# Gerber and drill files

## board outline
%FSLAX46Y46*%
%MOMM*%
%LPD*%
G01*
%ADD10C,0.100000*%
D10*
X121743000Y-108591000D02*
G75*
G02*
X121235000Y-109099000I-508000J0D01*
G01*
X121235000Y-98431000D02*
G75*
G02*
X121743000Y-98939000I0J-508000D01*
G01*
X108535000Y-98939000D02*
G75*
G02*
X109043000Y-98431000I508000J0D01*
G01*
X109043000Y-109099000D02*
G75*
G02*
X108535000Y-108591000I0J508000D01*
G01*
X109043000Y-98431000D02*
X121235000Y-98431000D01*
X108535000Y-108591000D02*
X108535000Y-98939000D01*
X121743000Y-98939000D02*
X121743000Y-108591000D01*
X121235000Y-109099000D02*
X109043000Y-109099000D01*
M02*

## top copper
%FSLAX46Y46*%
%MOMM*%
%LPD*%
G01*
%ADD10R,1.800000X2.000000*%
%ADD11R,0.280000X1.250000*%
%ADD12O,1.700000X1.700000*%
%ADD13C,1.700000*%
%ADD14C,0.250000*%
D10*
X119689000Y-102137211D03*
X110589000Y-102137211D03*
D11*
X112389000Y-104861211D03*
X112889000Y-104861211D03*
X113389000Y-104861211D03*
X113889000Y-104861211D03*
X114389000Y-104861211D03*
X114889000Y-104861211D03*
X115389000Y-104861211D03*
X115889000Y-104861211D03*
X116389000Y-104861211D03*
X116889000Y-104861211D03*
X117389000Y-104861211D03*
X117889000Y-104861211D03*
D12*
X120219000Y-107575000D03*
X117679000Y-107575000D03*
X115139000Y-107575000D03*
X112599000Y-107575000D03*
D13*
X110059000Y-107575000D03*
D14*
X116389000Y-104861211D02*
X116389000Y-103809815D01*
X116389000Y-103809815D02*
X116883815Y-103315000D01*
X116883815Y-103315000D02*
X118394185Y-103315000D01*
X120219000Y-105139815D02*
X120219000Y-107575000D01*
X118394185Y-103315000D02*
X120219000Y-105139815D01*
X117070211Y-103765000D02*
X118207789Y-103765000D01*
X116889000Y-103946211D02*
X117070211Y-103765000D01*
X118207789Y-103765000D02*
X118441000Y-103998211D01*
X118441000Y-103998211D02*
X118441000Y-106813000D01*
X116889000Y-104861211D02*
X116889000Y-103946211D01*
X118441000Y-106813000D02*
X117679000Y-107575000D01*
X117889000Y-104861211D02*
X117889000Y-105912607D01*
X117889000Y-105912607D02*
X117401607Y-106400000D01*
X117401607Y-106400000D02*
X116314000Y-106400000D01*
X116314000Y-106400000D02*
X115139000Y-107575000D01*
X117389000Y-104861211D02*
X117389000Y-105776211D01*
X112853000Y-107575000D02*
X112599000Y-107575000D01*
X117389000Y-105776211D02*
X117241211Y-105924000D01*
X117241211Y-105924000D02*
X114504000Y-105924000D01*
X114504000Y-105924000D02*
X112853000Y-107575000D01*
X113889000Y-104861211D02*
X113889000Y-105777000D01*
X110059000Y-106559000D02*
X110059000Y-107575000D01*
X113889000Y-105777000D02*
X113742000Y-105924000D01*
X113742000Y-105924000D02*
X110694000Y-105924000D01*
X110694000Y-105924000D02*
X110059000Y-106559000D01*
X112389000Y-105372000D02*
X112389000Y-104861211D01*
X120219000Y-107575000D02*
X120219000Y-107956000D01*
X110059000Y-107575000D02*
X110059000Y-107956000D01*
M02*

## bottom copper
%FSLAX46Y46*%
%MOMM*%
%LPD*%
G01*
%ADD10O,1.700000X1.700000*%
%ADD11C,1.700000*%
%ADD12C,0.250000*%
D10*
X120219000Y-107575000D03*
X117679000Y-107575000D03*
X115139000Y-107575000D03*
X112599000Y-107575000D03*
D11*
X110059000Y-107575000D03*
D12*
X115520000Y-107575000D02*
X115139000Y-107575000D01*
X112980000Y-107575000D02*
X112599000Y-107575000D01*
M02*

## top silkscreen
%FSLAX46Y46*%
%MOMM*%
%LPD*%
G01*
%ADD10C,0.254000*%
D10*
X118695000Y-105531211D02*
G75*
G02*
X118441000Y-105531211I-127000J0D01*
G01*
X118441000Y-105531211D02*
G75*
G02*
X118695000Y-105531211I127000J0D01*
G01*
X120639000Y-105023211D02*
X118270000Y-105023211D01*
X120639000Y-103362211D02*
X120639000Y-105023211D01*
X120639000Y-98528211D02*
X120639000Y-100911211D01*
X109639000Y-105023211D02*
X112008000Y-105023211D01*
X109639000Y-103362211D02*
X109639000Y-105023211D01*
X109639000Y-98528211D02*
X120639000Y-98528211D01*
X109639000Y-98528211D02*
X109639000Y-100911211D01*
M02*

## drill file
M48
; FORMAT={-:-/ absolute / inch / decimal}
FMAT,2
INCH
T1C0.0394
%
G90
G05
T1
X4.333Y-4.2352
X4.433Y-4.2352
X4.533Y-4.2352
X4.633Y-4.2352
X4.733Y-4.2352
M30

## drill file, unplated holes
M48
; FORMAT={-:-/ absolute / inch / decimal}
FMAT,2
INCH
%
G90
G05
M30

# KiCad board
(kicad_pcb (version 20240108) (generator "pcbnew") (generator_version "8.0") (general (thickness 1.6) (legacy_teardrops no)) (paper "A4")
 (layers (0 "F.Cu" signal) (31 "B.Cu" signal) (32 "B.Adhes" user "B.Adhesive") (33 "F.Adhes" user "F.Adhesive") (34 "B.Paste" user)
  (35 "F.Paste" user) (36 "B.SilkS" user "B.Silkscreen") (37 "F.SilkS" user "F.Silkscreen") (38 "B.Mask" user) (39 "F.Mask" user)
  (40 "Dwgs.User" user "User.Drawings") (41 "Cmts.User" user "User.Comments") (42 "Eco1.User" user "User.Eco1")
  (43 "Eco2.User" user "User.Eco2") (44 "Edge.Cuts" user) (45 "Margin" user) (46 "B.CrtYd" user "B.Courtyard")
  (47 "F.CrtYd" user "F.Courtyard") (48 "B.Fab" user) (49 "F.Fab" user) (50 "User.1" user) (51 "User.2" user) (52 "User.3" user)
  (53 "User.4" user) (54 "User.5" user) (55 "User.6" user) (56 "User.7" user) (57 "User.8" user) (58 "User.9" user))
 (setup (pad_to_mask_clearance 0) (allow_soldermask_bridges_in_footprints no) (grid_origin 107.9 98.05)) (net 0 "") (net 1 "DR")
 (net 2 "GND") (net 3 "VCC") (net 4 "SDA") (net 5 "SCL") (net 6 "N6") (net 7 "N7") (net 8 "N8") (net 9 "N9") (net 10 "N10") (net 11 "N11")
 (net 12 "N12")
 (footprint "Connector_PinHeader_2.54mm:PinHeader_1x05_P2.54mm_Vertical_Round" (layer "F.Cu") (at 110.059 107.575 90)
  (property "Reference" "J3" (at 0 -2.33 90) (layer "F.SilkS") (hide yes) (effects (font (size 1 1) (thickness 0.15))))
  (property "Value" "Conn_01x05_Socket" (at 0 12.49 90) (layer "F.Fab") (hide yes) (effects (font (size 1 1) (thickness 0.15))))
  (pad "1" thru_hole circle (at 0 0 90) (size 1.7 1.7) (drill 1) (layers "*.Cu" "*.Mask") (remove_unused_layers no) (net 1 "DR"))
  (pad "2" thru_hole oval (at 0 2.54 90) (size 1.7 1.7) (drill 1) (layers "*.Cu" "*.Mask") (remove_unused_layers no) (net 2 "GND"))
  (pad "3" thru_hole oval (at 0 5.08 90) (size 1.7 1.7) (drill 1) (layers "*.Cu" "*.Mask") (remove_unused_layers no) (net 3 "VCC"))
  (pad "4" thru_hole oval (at 0 7.62 90) (size 1.7 1.7) (drill 1) (layers "*.Cu" "*.Mask") (remove_unused_layers no) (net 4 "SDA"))
  (pad "5" thru_hole oval (at 0 10.16 90) (size 1.7 1.7) (drill 1) (layers "*.Cu" "*.Mask") (remove_unused_layers no) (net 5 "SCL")))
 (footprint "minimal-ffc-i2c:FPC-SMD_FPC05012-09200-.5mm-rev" (layer "F.Cu") (at 115.139 103.499211 180)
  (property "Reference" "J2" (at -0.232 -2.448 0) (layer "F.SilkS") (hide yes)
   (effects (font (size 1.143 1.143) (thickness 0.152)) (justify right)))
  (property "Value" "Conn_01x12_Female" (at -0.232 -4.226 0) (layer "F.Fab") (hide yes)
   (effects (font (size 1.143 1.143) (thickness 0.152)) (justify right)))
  (fp_line (start 5.5 4.971) (end 5.5 2.588) (stroke (width 0.254) (type solid)) (layer "F.SilkS"))
  (fp_line (start 5.5 4.971) (end -5.5 4.971) (stroke (width 0.254) (type solid)) (layer "F.SilkS"))
  (fp_line (start 5.5 0.137) (end 5.5 -1.524) (stroke (width 0.254) (type solid)) (layer "F.SilkS"))
  (fp_line (start 5.5 -1.524) (end 3.131 -1.524) (stroke (width 0.254) (type solid)) (layer "F.SilkS"))
  (fp_line (start -5.5 4.971) (end -5.5 2.588) (stroke (width 0.254) (type solid)) (layer "F.SilkS"))
  (fp_line (start -5.5 0.137) (end -5.5 -1.524) (stroke (width 0.254) (type solid)) (layer "F.SilkS"))
  (fp_line (start -5.5 -1.524) (end -3.131 -1.524) (stroke (width 0.254) (type solid)) (layer "F.SilkS"))
  (fp_circle (center -3.429 -2.032) (end -3.302 -2.032) (stroke (width 0.254) (type solid)) (fill none) (layer "F.SilkS"))
  (pad "1" smd rect (at -2.75 -1.362 180) (size 0.28 1.25) (layers "F.Cu" "F.Paste" "F.Mask") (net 3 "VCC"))
  (pad "2" smd rect (at -2.25 -1.362 180) (size 0.28 1.25) (layers "F.Cu" "F.Paste" "F.Mask") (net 2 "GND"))
  (pad "3" smd rect (at -1.75 -1.362 180) (size 0.28 1.25) (layers "F.Cu" "F.Paste" "F.Mask") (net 4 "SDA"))
  (pad "4" smd rect (at -1.25 -1.362 180) (size 0.28 1.25) (layers "F.Cu" "F.Paste" "F.Mask") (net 5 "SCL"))
  (pad "5" smd rect (at -0.75 -1.362 180) (size 0.28 1.25) (layers "F.Cu" "F.Paste" "F.Mask") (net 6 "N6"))
  (pad "6" smd rect (at -0.25 -1.362 180) (size 0.28 1.25) (layers "F.Cu" "F.Paste" "F.Mask") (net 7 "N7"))
  (pad "7" smd rect (at 0.25 -1.362 180) (size 0.28 1.25) (layers "F.Cu" "F.Paste" "F.Mask") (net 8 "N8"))
  (pad "8" smd rect (at 0.75 -1.362 180) (size 0.28 1.25) (layers "F.Cu" "F.Paste" "F.Mask") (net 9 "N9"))
  (pad "9" smd rect (at 1.25 -1.362 180) (size 0.28 1.25) (layers "F.Cu" "F.Paste" "F.Mask") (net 1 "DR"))
  (pad "10" smd rect (at 1.75 -1.362 180) (size 0.28 1.25) (layers "F.Cu" "F.Paste" "F.Mask") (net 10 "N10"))
  (pad "11" smd rect (at 2.25 -1.362 180) (size 0.28 1.25) (layers "F.Cu" "F.Paste" "F.Mask") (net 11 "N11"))
  (pad "12" smd rect (at 2.75 -1.362 180) (size 0.28 1.25) (layers "F.Cu" "F.Paste" "F.Mask") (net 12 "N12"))
  (pad "13" smd rect (at 4.55 1.362 180) (size 1.8 2) (layers "F.Cu" "F.Paste" "F.Mask"))
  (pad "14" smd rect (at -4.55 1.362 180) (size 1.8 2) (layers "F.Cu" "F.Paste" "F.Mask")))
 (gr_arc (start 121.743 108.591) (mid 121.59421 108.95021) (end 121.235 109.099) (stroke (width 0.1) (type default)) (layer "Edge.Cuts"))
 (gr_arc (start 121.235 98.431) (mid 121.59421 98.57979) (end 121.743 98.939) (stroke (width 0.1) (type default)) (layer "Edge.Cuts"))
 (gr_line (start 121.235 109.099) (end 109.043 109.099) (stroke (width 0.1) (type default)) (layer "Edge.Cuts"))
 (gr_arc (start 109.043 109.099) (mid 108.68379 108.95021) (end 108.535 108.591) (stroke (width 0.1) (type default)) (layer "Edge.Cuts"))
 (gr_line (start 109.043 98.431) (end 121.235 98.431) (stroke (width 0.1) (type default)) (layer "Edge.Cuts"))
 (gr_line (start 121.743 98.939) (end 121.743 108.591) (stroke (width 0.1) (type default)) (layer "Edge.Cuts"))
 (gr_line (start 108.535 108.591) (end 108.535 98.939) (stroke (width 0.1) (type default)) (layer "Edge.Cuts"))
 (gr_arc (start 108.535 98.939) (mid 108.68379 98.57979) (end 109.043 98.431) (stroke (width 0.1) (type default)) (layer "Edge.Cuts"))
 (segment (start 116.314 106.4) (end 115.139 107.575) (width 0.25) (layer "F.Cu") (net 3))
 (segment (start 117.401607 106.4) (end 116.314 106.4) (width 0.25) (layer "F.Cu") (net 3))
 (segment (start 117.889 105.912607) (end 117.401607 106.4) (width 0.25) (layer "F.Cu") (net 3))
 (segment (start 117.889 104.861211) (end 117.889 105.912607) (width 0.25) (layer "F.Cu") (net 3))
 (segment (start 115.52 107.575) (end 115.139 107.575) (width 0.25) (layer "B.Cu") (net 3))
 (segment (start 110.059 106.559) (end 110.059 107.575) (width 0.25) (layer "F.Cu") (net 1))
 (segment (start 110.694 105.924) (end 110.059 106.559) (width 0.25) (layer "F.Cu") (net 1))
 (segment (start 110.059 107.575) (end 110.059 107.956) (width 0.25) (layer "F.Cu") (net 1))
 (segment (start 113.889 105.777) (end 113.742 105.924) (width 0.25) (layer "F.Cu") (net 1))
 (segment (start 113.889 104.861211) (end 113.889 105.777) (width 0.25) (layer "F.Cu") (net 1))
 (segment (start 113.742 105.924) (end 110.694 105.924) (width 0.25) (layer "F.Cu") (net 1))
 (segment (start 116.889 103.946211) (end 117.070211 103.765) (width 0.25) (layer "F.Cu") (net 4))
 (segment (start 118.441 103.998211) (end 118.441 106.813) (width 0.25) (layer "F.Cu") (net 4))
 (segment (start 118.207789 103.765) (end 118.441 103.998211) (width 0.25) (layer "F.Cu") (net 4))
 (segment (start 118.441 106.813) (end 117.679 107.575) (width 0.25) (layer "F.Cu") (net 4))
 (segment (start 116.889 104.861211) (end 116.889 103.946211) (width 0.25) (layer "F.Cu") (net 4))
 (segment (start 117.070211 103.765) (end 118.207789 103.765) (width 0.25) (layer "F.Cu") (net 4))
 (segment (start 120.219 105.139815) (end 120.219 107.575) (width 0.25) (layer "F.Cu") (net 5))
 (segment (start 116.883815 103.315) (end 118.394185 103.315) (width 0.25) (layer "F.Cu") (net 5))
 (segment (start 116.389 103.809815) (end 116.883815 103.315) (width 0.25) (layer "F.Cu") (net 5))
 (segment (start 118.394185 103.315) (end 120.219 105.139815) (width 0.25) (layer "F.Cu") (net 5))
 (segment (start 116.389 104.861211) (end 116.389 103.809815) (width 0.25) (layer "F.Cu") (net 5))
 (segment (start 120.219 107.575) (end 120.219 107.956) (width 0.25) (layer "F.Cu") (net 5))
 (segment (start 117.389 104.861211) (end 117.389 105.776211) (width 0.25) (layer "F.Cu") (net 2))
 (segment (start 117.241211 105.924) (end 114.504 105.924) (width 0.25) (layer "F.Cu") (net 2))
 (segment (start 117.389 105.776211) (end 117.241211 105.924) (width 0.25) (layer "F.Cu") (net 2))
 (segment (start 114.504 105.924) (end 112.853 107.575) (width 0.25) (layer "F.Cu") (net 2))
 (segment (start 112.853 107.575) (end 112.599 107.575) (width 0.25) (layer "F.Cu") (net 2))
 (segment (start 112.98 107.575) (end 112.599 107.575) (width 0.25) (layer "B.Cu") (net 2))
 (segment (start 112.389 105.372) (end 112.389 104.861211) (width 0.25) (layer "F.Cu") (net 12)))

